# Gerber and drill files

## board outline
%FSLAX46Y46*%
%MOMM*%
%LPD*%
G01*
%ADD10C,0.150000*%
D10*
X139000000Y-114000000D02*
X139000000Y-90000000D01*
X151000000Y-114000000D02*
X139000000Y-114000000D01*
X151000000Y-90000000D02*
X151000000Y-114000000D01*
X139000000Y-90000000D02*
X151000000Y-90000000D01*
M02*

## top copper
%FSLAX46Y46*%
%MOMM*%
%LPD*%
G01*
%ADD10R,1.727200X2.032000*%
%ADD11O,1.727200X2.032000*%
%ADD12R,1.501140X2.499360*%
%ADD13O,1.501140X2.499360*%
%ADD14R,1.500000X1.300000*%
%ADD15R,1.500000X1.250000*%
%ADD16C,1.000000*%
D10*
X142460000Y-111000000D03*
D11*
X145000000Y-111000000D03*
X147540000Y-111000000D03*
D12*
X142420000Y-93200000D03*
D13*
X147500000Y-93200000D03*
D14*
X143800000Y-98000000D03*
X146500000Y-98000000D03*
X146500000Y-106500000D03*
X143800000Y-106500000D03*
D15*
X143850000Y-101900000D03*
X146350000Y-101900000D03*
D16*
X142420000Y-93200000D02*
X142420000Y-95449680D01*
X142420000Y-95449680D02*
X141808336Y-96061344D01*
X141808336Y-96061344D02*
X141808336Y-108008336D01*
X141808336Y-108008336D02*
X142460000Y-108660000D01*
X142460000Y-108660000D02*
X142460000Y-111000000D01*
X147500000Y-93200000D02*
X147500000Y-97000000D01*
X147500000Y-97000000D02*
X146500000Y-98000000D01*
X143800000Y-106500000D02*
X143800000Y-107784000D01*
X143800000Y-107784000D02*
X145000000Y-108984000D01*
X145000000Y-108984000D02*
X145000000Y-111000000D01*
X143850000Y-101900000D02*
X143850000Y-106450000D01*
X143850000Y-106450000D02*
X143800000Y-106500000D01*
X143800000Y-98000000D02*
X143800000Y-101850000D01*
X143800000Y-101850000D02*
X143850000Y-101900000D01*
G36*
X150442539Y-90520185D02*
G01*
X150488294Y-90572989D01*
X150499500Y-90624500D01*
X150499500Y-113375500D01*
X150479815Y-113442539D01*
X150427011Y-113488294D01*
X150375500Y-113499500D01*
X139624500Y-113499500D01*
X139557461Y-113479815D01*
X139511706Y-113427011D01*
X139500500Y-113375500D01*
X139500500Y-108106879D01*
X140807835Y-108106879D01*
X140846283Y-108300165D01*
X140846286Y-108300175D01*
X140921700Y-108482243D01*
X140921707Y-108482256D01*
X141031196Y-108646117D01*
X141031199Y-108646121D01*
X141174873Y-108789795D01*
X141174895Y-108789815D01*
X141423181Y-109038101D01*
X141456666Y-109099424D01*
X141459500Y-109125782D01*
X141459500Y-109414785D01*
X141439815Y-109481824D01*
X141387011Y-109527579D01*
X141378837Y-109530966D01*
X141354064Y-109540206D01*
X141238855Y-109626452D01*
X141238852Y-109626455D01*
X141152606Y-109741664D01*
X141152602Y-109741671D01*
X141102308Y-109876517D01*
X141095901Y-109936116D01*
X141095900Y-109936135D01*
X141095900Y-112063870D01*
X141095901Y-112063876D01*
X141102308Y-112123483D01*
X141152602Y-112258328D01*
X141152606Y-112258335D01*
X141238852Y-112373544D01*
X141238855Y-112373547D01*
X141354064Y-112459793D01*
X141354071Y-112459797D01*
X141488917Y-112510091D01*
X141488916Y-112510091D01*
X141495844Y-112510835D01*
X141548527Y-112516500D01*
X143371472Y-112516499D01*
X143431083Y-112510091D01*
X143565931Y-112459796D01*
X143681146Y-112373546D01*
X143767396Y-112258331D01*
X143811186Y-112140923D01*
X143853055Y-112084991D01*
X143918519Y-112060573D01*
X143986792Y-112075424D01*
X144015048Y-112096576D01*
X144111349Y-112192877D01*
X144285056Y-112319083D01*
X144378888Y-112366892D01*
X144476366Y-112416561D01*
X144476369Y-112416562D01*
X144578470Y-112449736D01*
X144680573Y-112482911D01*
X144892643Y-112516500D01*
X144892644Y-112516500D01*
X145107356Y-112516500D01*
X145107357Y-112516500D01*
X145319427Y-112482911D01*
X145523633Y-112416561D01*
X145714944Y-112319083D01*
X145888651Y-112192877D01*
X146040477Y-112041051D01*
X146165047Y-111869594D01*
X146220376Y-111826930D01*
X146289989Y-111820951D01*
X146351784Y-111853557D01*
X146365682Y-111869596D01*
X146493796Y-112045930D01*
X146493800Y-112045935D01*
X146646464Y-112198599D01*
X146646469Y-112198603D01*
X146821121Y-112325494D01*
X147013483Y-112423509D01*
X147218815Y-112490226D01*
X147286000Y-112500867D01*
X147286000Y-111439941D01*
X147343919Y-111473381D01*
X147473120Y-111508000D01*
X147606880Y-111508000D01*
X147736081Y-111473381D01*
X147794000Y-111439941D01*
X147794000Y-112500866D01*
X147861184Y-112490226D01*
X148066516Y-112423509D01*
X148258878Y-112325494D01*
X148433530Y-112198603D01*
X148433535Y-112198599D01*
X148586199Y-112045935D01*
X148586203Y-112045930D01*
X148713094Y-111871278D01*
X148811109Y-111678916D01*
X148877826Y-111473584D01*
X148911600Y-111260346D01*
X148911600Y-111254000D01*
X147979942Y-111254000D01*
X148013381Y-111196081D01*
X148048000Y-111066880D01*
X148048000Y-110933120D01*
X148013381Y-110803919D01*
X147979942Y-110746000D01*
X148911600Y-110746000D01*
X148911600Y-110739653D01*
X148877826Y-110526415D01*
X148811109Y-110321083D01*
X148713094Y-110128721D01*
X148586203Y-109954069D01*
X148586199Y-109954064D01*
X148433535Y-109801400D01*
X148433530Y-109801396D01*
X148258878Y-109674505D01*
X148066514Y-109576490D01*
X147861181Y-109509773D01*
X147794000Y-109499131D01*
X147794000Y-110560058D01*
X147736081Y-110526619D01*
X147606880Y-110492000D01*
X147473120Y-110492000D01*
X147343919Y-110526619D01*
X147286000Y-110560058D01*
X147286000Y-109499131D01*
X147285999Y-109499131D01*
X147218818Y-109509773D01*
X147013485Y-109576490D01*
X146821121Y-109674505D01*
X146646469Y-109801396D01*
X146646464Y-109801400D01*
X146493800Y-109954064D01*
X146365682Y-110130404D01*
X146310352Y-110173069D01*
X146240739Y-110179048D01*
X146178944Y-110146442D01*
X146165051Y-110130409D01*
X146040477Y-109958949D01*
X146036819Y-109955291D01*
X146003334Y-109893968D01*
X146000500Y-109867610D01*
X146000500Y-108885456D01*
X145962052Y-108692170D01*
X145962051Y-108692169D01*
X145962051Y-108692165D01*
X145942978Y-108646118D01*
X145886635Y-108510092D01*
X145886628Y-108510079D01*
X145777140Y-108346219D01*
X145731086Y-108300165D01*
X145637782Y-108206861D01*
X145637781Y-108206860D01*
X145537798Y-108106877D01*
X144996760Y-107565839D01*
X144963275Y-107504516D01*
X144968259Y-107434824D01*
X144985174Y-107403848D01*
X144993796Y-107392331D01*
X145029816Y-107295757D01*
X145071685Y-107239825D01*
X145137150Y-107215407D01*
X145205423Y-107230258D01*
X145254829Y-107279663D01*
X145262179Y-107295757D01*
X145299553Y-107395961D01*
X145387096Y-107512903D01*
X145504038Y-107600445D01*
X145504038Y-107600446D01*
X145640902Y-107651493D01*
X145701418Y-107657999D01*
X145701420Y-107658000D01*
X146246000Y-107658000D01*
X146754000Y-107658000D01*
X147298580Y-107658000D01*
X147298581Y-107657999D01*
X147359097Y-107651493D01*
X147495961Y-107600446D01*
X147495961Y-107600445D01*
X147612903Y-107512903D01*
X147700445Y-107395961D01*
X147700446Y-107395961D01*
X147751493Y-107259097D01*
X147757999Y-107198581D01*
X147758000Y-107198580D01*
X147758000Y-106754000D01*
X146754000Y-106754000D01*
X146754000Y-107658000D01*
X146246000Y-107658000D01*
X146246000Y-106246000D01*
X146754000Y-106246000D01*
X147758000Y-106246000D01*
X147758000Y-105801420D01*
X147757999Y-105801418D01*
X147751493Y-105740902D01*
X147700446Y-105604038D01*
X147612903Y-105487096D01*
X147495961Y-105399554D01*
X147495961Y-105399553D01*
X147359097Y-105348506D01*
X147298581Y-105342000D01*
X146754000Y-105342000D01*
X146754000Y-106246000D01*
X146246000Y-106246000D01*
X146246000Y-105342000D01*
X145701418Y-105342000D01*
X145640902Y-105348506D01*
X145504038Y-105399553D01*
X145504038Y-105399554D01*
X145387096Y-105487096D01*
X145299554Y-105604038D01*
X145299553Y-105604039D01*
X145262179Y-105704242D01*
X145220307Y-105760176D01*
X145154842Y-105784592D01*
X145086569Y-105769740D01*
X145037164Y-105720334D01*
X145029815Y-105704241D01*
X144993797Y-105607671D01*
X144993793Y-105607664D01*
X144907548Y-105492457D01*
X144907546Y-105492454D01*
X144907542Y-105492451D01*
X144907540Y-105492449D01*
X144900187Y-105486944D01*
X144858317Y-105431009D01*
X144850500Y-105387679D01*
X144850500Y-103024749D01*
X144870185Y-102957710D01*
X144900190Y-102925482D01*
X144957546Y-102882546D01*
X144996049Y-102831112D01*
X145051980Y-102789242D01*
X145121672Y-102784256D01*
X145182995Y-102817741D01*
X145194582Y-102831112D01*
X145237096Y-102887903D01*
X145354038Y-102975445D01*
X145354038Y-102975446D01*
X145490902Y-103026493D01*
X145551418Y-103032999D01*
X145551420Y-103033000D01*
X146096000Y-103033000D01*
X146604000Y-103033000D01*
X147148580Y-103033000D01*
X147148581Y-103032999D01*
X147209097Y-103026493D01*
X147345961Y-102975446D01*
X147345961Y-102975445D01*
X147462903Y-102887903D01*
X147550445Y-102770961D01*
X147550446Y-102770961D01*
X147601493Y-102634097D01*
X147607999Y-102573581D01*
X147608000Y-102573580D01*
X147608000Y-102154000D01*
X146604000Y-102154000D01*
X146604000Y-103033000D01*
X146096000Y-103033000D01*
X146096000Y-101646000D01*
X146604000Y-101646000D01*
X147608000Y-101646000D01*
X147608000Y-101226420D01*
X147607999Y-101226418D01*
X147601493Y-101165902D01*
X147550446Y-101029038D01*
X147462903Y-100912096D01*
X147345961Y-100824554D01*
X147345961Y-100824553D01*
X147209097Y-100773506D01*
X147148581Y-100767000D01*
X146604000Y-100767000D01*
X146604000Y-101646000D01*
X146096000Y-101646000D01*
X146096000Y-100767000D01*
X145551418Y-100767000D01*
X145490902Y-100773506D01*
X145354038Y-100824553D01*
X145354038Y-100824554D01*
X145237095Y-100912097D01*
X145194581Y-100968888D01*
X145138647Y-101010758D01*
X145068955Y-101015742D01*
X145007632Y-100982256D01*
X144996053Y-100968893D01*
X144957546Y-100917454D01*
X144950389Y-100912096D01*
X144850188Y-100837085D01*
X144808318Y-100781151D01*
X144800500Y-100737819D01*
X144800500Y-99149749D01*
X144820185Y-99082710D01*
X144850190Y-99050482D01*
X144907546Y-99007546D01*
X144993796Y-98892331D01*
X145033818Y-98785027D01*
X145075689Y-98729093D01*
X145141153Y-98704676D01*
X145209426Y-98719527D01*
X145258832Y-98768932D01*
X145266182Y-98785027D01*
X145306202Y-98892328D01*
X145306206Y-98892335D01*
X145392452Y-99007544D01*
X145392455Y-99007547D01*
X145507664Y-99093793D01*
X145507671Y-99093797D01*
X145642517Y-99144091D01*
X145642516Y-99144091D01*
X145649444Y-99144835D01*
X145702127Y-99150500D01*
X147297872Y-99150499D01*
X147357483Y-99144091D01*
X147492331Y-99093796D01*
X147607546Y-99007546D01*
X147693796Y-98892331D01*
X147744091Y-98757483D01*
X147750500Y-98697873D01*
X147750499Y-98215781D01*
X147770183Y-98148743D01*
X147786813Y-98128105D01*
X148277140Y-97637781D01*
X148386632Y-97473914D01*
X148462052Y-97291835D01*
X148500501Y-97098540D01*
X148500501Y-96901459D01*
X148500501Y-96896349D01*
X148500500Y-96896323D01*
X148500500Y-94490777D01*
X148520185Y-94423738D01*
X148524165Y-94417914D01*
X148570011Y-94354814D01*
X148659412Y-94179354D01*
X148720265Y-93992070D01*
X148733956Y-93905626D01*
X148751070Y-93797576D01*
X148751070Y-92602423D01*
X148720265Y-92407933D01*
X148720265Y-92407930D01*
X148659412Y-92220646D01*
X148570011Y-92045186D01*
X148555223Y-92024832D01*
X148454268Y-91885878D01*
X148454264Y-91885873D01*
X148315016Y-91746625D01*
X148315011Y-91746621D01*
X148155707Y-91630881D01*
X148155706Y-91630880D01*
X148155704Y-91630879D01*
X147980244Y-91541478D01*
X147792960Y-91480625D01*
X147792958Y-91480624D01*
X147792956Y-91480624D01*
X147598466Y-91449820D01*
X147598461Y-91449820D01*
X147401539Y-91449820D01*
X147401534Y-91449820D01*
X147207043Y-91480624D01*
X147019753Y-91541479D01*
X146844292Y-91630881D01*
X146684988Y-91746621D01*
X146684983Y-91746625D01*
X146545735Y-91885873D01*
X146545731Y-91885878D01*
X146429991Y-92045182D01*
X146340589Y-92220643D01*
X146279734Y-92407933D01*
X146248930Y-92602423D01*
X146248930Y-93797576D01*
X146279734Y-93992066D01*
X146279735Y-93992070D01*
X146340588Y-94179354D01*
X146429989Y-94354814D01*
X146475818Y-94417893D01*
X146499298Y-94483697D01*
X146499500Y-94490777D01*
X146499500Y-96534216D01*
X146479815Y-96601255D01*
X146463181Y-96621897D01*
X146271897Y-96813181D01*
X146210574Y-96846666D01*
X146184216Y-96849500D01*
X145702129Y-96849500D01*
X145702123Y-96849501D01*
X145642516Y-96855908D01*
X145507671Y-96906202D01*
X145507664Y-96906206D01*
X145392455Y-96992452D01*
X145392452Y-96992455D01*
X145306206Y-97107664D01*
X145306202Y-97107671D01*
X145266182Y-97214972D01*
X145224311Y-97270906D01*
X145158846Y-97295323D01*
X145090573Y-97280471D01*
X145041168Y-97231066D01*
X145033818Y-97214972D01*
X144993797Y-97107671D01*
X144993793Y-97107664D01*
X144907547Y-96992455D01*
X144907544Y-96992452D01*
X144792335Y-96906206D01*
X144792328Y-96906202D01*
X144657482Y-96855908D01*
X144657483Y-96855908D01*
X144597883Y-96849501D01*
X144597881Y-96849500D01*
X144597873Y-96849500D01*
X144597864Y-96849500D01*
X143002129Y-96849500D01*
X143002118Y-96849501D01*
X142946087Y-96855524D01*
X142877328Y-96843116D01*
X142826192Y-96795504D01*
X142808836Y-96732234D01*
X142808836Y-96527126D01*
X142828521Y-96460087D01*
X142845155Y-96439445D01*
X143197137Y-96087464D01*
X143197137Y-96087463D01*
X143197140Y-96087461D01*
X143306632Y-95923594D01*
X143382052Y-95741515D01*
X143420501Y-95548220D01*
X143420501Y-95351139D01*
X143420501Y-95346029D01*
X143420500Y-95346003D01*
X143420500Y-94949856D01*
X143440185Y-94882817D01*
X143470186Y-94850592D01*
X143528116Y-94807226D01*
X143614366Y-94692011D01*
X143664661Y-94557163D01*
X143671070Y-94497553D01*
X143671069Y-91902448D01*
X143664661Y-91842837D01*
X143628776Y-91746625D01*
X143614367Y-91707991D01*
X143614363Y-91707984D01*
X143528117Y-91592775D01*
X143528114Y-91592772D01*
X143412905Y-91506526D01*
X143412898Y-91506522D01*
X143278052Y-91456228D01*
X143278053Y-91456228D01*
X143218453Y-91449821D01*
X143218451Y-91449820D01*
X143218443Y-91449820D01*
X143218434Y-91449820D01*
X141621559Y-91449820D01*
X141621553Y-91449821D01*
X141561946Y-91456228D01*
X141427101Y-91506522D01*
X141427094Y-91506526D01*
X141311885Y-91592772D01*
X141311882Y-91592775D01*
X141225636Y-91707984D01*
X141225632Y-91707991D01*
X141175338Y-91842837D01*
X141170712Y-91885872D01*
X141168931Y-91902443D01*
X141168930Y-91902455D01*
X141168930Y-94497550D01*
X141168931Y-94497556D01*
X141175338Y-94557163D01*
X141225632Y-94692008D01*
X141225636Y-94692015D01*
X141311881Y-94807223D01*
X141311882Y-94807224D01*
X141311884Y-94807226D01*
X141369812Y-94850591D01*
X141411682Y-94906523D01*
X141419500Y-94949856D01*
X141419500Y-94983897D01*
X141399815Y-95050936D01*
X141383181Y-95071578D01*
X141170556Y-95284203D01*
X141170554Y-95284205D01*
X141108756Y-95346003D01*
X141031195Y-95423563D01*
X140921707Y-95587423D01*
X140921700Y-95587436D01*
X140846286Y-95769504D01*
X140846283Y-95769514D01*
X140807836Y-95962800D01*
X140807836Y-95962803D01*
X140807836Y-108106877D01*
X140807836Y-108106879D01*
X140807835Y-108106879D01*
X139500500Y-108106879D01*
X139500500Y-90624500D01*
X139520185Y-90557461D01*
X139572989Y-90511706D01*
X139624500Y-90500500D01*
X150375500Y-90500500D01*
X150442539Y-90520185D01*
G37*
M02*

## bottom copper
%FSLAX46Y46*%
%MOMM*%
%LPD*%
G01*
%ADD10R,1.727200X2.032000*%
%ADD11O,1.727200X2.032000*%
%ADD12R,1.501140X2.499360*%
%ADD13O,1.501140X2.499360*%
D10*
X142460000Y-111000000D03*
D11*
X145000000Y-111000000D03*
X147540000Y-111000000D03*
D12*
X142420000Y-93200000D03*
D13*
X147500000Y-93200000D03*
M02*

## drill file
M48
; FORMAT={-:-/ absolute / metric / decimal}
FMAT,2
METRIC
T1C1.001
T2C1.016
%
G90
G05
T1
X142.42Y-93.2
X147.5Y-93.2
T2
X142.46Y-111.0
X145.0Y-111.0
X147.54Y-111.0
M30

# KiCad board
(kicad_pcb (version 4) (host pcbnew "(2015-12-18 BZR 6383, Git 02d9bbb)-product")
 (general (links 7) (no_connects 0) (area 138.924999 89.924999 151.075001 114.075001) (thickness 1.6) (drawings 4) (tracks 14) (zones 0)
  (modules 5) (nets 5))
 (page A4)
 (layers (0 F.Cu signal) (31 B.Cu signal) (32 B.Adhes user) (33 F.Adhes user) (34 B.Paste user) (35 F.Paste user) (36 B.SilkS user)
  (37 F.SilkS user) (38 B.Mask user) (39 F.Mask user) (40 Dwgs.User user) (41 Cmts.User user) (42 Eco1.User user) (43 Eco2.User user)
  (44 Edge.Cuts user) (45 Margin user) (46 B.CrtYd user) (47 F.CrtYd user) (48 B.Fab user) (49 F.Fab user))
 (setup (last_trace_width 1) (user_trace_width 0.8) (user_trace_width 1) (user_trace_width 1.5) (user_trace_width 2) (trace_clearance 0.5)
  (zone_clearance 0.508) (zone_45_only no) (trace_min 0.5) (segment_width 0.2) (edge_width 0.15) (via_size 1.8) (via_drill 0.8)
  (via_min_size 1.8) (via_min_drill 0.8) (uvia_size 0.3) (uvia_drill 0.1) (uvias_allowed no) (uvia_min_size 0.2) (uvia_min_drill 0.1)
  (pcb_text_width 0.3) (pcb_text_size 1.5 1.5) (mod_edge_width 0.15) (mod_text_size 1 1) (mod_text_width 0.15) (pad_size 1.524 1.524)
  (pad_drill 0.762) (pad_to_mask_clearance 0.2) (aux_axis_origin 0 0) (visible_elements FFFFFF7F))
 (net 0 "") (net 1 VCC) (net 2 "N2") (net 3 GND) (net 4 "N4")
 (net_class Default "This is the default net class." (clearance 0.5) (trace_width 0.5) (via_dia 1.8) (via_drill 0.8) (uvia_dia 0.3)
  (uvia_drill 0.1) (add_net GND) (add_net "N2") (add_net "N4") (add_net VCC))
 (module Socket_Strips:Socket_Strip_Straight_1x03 (layer F.Cu) (at 142.46 111)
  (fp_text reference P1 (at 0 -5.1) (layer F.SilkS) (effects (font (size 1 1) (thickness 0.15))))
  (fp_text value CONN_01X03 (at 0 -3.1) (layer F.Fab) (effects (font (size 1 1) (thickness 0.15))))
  (pad 1 thru_hole rect (at 0 0) (size 1.7272 2.032) (drill 1.016) (layers *.Cu *.Mask F.SilkS) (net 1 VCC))
  (pad 2 thru_hole oval (at 2.54 0) (size 1.7272 2.032) (drill 1.016) (layers *.Cu *.Mask F.SilkS) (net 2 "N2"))
  (pad 3 thru_hole oval (at 5.08 0) (size 1.7272 2.032) (drill 1.016) (layers *.Cu *.Mask F.SilkS) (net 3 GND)))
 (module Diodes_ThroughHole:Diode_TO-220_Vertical (layer F.Cu) (at 142.42 93.2)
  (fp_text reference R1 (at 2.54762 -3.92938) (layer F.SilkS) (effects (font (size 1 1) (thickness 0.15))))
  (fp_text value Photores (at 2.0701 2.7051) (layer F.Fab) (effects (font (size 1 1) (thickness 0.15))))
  (pad 1 thru_hole rect (at 0 0 90) (size 2.49936 1.50114) (drill 1.00076) (layers *.Cu *.Mask F.SilkS) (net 1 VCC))
  (pad 2 thru_hole oval (at 5.08 0 90) (size 2.49936 1.50114) (drill 1.00076) (layers *.Cu *.Mask F.SilkS) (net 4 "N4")))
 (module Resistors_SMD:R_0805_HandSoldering (layer F.Cu) (at 145.15 98)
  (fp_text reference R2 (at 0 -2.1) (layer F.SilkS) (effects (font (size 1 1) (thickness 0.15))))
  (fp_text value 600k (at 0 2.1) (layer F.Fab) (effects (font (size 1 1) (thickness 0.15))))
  (pad 1 smd rect (at -1.35 0) (size 1.5 1.3) (layers F.Cu F.Paste F.Mask) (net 2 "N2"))
  (pad 2 smd rect (at 1.35 0) (size 1.5 1.3) (layers F.Cu F.Paste F.Mask) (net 4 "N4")))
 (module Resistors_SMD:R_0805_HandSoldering (layer F.Cu) (at 145.15 106.5 180)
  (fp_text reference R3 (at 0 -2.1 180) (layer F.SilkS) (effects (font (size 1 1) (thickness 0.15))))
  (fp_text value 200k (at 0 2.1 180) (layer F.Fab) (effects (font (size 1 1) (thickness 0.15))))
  (pad 1 smd rect (at -1.35 0 180) (size 1.5 1.3) (layers F.Cu F.Paste F.Mask) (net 3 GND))
  (pad 2 smd rect (at 1.35 0 180) (size 1.5 1.3) (layers F.Cu F.Paste F.Mask) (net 2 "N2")))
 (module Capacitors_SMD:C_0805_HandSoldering (layer F.Cu) (at 145.1 101.9)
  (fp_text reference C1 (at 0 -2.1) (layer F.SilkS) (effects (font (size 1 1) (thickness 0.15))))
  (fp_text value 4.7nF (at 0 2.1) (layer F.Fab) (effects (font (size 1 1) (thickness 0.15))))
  (pad 1 smd rect (at -1.25 0) (size 1.5 1.25) (layers F.Cu F.Paste F.Mask) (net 2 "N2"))
  (pad 2 smd rect (at 1.25 0) (size 1.5 1.25) (layers F.Cu F.Paste F.Mask) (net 3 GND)))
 (gr_line (start 139 114) (end 139 90) (layer Edge.Cuts) (width 0.15))
 (gr_line (start 151 114) (end 139 114) (layer Edge.Cuts) (width 0.15))
 (gr_line (start 151 90) (end 151 114) (layer Edge.Cuts) (width 0.15))
 (gr_line (start 139 90) (end 151 90) (layer Edge.Cuts) (width 0.15))
 (segment (start 142.42 93.2) (end 142.42 95.44968) (width 1) (layer F.Cu) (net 1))
 (segment (start 142.42 95.44968) (end 141.808336 96.061344) (width 1) (layer F.Cu) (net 1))
 (segment (start 141.808336 96.061344) (end 141.808336 108.008336) (width 1) (layer F.Cu) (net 1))
 (segment (start 141.808336 108.008336) (end 142.46 108.66) (width 1) (layer F.Cu) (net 1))
 (segment (start 142.46 108.66) (end 142.46 111) (width 1) (layer F.Cu) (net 1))
 (segment (start 147.5 93.2) (end 147.5 97) (width 1) (layer F.Cu) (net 4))
 (segment (start 147.5 97) (end 146.5 98) (width 1) (layer F.Cu) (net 4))
 (segment (start 143.8 106.5) (end 143.8 107.784) (width 1) (layer F.Cu) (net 2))
 (segment (start 143.8 107.784) (end 145 108.984) (width 1) (layer F.Cu) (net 2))
 (segment (start 145 108.984) (end 145 111) (width 1) (layer F.Cu) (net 2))
 (segment (start 143.85 101.9) (end 143.85 106.45) (width 1) (layer F.Cu) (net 2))
 (segment (start 143.85 106.45) (end 143.8 106.5) (width 1) (layer F.Cu) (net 2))
 (segment (start 143.8 98) (end 143.8 101.85) (width 1) (layer F.Cu) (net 2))
 (segment (start 143.8 101.85) (end 143.85 101.9) (width 1) (layer F.Cu) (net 2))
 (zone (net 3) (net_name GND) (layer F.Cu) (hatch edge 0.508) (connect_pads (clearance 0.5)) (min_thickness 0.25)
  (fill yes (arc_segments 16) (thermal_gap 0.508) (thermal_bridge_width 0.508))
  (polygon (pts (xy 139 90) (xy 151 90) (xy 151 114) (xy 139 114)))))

